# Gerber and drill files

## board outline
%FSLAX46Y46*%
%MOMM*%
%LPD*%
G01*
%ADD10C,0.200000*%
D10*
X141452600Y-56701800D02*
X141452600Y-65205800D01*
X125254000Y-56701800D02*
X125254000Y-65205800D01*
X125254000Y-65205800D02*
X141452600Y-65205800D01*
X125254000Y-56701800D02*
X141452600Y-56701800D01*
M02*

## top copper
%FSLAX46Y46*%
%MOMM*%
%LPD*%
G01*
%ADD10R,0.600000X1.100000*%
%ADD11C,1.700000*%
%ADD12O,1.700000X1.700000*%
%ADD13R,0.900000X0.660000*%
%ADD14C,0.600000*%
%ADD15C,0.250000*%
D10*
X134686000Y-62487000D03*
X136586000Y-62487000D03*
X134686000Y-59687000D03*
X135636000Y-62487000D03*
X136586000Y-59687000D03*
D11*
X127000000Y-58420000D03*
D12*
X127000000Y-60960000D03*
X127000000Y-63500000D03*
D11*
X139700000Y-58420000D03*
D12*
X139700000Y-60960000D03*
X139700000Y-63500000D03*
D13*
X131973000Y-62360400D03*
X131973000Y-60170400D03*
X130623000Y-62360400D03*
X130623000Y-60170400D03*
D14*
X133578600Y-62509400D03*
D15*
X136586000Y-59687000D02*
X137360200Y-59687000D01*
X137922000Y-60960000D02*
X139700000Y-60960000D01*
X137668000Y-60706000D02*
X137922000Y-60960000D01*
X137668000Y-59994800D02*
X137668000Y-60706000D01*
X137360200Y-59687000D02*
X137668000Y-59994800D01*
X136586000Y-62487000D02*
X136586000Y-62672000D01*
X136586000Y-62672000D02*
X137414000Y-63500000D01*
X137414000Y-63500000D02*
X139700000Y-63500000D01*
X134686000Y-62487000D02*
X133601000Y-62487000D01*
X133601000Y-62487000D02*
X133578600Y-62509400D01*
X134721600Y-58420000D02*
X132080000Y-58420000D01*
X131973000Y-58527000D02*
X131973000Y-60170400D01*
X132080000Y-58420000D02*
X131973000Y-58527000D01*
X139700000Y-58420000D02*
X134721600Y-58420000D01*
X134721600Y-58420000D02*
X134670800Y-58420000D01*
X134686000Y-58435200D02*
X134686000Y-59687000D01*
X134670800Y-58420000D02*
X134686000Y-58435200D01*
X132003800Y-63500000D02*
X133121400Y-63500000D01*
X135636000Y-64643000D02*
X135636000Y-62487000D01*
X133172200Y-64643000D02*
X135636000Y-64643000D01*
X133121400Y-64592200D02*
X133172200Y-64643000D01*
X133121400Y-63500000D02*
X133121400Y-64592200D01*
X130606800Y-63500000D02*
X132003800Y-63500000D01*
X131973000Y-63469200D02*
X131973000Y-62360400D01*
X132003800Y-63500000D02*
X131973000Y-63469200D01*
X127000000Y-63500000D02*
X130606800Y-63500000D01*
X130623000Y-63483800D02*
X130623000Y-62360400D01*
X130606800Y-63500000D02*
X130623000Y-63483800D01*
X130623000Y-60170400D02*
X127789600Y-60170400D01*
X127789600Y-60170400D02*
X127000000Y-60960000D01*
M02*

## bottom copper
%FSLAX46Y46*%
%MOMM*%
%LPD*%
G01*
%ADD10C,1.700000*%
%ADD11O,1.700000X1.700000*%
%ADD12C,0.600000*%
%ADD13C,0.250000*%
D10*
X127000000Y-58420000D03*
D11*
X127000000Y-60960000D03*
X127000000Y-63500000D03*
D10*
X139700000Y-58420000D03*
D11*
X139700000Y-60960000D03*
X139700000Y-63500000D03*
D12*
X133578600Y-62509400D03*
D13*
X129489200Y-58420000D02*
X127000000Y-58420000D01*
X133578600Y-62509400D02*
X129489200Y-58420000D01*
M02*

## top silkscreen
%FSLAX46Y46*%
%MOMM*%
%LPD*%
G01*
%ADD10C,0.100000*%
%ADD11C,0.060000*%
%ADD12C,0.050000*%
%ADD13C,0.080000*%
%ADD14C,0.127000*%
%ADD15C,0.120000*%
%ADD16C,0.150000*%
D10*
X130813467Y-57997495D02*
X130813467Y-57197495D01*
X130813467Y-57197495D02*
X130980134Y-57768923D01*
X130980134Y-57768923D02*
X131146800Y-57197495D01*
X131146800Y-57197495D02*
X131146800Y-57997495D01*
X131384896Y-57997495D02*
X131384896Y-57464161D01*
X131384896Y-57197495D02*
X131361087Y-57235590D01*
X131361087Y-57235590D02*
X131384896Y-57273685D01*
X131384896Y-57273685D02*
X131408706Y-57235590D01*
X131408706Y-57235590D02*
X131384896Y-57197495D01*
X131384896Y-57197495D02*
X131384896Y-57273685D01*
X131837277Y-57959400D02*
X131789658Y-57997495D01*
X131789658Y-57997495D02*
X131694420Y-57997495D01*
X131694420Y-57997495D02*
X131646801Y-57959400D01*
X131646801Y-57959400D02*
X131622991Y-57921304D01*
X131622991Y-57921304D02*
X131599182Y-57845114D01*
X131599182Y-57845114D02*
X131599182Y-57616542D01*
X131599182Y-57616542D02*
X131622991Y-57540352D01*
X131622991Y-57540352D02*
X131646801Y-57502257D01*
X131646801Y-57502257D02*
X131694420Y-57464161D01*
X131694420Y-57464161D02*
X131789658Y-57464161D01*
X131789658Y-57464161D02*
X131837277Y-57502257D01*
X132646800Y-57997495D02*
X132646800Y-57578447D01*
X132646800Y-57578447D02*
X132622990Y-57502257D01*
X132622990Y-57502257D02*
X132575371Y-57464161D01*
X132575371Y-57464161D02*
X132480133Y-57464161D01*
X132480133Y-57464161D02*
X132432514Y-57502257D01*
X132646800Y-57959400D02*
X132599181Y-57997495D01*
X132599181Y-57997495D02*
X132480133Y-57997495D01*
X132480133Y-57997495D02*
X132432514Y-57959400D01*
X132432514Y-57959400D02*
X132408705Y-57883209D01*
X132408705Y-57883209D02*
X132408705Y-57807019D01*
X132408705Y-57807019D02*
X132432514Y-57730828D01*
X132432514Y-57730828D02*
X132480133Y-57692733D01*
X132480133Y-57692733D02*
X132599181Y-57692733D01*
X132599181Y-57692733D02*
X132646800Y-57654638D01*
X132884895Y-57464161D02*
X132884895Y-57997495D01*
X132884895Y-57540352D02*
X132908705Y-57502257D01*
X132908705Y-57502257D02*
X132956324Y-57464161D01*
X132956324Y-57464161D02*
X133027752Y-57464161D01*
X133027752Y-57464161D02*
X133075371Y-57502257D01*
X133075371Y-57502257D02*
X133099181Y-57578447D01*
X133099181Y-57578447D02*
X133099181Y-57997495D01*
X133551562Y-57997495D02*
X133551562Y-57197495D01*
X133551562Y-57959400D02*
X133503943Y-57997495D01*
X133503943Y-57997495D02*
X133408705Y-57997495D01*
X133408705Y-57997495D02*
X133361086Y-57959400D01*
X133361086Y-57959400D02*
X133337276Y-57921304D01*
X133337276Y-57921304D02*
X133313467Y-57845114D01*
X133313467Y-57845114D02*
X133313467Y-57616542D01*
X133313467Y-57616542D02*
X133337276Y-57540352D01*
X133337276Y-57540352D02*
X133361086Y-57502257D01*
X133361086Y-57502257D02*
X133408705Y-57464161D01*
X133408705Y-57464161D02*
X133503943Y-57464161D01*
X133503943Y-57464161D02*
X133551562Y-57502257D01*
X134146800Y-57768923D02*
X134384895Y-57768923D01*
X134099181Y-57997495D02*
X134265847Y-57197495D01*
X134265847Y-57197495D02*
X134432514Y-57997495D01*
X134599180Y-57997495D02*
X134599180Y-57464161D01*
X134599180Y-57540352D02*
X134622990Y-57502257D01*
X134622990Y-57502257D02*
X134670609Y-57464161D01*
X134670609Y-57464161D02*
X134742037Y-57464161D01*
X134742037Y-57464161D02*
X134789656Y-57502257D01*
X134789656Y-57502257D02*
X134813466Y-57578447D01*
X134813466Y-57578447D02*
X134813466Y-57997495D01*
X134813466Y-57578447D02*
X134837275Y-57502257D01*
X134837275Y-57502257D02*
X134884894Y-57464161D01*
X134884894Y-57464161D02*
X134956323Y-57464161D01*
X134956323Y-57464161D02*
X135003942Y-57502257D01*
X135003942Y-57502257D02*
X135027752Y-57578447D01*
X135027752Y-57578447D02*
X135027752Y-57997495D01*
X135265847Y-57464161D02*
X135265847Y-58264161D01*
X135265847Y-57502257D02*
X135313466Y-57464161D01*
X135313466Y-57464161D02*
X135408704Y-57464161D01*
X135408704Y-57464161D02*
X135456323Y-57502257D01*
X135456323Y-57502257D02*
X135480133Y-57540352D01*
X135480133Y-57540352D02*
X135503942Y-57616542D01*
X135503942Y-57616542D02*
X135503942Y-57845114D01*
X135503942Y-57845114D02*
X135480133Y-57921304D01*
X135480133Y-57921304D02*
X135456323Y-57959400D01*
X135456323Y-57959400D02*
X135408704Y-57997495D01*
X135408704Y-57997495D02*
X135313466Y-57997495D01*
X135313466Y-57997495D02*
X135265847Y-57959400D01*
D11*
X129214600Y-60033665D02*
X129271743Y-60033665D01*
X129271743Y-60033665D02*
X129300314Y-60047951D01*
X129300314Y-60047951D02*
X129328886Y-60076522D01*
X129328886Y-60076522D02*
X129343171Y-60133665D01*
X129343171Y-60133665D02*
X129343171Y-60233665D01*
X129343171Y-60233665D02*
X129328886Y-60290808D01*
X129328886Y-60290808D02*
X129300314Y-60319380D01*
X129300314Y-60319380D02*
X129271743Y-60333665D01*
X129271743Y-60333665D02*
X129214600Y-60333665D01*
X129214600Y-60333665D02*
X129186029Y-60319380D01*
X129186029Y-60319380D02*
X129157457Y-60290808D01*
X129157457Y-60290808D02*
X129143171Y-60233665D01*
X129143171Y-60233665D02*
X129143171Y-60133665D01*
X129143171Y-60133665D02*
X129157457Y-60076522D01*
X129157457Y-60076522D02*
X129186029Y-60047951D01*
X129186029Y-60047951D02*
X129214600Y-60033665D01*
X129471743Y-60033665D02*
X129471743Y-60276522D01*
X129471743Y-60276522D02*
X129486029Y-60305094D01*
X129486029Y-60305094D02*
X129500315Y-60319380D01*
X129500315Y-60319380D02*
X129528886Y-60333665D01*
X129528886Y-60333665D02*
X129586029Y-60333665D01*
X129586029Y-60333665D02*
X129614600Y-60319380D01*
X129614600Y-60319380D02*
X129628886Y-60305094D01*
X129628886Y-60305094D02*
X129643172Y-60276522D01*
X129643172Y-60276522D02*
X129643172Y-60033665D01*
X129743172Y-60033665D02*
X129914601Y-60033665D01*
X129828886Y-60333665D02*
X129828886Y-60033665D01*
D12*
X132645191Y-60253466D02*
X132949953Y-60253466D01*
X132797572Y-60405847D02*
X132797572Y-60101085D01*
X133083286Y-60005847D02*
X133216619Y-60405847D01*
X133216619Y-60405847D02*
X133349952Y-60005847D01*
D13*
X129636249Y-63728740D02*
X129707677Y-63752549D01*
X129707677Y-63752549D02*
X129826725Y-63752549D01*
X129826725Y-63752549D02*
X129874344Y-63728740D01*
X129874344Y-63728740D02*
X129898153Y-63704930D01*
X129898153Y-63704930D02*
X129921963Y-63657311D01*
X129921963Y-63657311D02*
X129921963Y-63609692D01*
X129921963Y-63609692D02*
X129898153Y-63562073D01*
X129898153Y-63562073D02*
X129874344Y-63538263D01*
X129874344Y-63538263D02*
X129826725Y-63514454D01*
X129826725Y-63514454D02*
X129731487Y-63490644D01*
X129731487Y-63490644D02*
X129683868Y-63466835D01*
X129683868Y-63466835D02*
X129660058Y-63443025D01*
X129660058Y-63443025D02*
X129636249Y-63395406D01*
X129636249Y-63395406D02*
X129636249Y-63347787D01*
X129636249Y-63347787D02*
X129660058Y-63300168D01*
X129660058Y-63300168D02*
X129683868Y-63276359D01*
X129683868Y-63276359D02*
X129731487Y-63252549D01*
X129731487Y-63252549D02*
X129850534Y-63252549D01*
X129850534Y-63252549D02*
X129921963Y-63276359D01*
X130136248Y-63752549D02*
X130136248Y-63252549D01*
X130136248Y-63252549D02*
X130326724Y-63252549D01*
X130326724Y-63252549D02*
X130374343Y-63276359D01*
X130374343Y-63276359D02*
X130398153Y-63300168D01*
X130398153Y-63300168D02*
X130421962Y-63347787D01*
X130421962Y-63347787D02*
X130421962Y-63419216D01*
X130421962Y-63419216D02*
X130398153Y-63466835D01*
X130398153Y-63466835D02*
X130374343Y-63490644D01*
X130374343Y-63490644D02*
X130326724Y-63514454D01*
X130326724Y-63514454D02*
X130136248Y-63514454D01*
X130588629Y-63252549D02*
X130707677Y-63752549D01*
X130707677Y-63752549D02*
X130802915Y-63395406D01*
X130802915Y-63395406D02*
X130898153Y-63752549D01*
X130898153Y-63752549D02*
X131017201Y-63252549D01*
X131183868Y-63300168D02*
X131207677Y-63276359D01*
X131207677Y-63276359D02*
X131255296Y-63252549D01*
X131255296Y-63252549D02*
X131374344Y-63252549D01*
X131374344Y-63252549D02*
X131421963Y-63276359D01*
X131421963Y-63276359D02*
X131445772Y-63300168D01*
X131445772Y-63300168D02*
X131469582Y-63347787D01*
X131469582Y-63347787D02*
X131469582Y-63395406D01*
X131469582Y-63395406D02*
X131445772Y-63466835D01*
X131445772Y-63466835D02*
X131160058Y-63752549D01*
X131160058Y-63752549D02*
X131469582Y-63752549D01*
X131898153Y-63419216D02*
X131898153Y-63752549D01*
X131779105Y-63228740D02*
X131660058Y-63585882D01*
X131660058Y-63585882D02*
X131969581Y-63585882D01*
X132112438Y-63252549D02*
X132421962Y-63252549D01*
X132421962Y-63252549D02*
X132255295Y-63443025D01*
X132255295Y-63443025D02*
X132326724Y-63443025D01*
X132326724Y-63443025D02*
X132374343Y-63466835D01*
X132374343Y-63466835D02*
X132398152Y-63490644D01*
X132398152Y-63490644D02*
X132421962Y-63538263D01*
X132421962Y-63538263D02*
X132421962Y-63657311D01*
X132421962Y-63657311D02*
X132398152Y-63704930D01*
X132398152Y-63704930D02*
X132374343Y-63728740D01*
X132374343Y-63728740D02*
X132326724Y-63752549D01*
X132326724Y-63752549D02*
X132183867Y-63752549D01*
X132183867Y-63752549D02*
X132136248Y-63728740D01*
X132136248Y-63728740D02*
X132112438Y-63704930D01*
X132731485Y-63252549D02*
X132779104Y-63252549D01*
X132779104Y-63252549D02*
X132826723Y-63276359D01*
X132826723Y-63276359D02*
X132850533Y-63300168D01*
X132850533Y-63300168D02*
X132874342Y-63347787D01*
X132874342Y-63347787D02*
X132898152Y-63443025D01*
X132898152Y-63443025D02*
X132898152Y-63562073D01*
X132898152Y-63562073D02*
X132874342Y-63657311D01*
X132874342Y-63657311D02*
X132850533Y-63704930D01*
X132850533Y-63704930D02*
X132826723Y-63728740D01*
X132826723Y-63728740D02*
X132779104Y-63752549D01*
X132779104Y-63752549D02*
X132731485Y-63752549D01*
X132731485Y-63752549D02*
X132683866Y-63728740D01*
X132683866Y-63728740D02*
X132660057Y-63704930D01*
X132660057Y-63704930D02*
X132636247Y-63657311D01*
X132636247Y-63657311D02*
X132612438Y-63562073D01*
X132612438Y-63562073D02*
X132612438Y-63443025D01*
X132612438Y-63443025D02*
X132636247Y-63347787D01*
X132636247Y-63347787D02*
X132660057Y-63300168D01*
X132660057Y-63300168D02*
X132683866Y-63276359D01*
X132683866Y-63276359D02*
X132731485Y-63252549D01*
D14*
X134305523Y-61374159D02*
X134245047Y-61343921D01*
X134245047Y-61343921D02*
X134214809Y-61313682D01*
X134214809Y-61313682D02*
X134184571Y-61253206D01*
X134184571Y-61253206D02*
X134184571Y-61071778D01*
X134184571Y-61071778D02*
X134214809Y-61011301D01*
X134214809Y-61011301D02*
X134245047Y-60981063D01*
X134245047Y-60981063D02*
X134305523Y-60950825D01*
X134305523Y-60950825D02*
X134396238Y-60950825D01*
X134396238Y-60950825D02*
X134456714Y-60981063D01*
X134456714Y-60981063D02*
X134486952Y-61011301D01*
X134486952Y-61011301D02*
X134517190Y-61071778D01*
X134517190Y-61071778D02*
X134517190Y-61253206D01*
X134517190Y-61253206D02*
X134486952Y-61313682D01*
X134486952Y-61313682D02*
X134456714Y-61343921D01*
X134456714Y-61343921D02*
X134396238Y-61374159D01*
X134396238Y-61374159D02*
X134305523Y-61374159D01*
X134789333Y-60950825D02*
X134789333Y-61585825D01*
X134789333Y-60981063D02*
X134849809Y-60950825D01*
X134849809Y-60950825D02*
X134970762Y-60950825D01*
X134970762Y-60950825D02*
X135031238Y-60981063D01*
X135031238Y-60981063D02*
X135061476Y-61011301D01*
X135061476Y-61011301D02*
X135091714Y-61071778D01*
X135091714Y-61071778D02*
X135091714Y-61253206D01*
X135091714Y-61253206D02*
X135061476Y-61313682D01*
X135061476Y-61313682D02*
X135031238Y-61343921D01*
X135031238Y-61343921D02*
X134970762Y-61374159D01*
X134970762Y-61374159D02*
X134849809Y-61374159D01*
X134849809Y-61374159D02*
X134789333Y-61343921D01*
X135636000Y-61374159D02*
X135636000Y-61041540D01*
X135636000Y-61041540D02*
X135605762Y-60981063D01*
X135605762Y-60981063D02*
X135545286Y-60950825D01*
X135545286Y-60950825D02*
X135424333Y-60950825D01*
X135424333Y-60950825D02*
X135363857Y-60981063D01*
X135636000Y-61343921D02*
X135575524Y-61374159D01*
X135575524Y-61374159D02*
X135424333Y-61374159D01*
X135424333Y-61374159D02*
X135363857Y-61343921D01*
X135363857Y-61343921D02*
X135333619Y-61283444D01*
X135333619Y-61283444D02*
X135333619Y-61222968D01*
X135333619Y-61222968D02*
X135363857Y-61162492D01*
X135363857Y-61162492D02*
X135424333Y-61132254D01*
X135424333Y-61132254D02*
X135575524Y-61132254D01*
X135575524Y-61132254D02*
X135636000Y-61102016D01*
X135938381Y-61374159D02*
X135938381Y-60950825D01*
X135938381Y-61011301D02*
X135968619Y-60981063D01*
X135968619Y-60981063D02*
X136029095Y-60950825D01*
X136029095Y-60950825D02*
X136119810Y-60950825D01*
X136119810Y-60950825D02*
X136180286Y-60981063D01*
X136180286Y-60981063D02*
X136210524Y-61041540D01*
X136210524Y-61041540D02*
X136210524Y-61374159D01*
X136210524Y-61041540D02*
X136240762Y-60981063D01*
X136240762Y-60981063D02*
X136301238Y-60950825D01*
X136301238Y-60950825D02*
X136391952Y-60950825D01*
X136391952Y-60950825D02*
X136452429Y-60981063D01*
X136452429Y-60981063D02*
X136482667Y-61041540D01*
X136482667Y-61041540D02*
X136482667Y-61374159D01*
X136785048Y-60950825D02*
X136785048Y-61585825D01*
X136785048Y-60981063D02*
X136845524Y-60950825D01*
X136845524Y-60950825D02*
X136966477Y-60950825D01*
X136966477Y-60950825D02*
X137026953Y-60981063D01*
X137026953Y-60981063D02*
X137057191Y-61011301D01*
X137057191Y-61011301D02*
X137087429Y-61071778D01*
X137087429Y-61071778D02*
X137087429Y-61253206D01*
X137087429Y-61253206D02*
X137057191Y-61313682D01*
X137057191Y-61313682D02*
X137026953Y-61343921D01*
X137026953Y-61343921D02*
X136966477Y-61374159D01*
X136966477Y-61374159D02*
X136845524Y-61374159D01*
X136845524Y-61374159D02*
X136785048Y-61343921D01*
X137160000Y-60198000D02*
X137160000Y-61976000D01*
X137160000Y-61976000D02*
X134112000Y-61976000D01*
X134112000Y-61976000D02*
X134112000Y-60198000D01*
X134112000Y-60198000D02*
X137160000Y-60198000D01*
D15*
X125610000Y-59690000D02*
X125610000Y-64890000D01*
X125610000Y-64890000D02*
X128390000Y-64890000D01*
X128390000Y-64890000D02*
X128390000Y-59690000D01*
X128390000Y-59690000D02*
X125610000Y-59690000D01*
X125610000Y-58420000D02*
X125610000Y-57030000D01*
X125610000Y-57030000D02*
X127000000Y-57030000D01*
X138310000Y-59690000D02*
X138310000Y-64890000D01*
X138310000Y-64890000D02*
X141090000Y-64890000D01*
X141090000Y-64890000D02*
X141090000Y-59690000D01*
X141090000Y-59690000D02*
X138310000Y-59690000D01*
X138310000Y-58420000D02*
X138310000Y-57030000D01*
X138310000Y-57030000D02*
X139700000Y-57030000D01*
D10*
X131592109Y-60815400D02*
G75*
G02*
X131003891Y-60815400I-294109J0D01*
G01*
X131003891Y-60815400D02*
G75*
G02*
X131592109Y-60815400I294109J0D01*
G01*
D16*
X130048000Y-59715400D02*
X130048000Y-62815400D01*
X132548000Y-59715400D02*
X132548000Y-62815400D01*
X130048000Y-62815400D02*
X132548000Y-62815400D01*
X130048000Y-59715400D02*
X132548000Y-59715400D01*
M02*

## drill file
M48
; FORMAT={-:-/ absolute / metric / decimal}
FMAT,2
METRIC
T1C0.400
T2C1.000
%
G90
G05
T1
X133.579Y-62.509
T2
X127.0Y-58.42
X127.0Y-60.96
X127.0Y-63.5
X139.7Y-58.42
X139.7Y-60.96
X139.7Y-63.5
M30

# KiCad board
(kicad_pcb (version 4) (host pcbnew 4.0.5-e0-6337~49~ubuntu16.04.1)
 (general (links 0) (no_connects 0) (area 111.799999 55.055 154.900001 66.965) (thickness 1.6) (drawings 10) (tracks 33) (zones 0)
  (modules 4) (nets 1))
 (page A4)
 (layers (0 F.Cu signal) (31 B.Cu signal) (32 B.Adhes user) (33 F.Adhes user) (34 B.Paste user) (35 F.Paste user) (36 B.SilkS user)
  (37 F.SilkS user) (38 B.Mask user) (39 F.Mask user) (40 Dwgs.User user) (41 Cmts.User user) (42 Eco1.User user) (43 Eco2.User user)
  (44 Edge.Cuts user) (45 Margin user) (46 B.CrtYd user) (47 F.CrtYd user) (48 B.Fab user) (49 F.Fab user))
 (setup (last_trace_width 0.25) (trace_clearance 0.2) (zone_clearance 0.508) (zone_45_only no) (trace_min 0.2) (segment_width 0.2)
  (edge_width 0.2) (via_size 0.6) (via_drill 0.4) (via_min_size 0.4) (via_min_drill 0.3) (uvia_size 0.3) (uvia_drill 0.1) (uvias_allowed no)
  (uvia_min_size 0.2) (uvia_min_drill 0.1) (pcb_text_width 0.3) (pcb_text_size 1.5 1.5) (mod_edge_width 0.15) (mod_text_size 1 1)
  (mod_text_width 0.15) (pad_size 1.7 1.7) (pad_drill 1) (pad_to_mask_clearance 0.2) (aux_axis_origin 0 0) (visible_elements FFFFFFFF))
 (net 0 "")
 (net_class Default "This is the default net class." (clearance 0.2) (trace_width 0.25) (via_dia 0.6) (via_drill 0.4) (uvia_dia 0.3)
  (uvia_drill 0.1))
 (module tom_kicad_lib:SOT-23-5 (layer F.Cu) (at 135.636 61.087) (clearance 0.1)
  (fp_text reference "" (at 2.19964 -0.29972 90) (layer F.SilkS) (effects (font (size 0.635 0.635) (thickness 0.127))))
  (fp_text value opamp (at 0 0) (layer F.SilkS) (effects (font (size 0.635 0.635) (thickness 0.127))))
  (fp_line (start 1.524 -0.889) (end 1.524 0.889) (layer F.SilkS) (width 0.127))
  (fp_line (start 1.524 0.889) (end -1.524 0.889) (layer F.SilkS) (width 0.127))
  (fp_line (start -1.524 0.889) (end -1.524 -0.889) (layer F.SilkS) (width 0.127))
  (fp_line (start -1.524 -0.889) (end 1.524 -0.889) (layer F.SilkS) (width 0.127))
  (pad 1 smd rect (at -0.95 1.4) (size 0.6 1.1) (layers F.Cu F.Paste F.Mask))
  (pad 3 smd rect (at 0.95 1.4) (size 0.6 1.1) (layers F.Cu F.Paste F.Mask))
  (pad 5 smd rect (at -0.95 -1.4) (size 0.6 1.1) (layers F.Cu F.Paste F.Mask))
  (pad 2 smd rect (at 0 1.4) (size 0.6 1.1) (layers F.Cu F.Paste F.Mask))
  (pad 4 smd rect (at 0.95 -1.4) (size 0.6 1.1) (layers F.Cu F.Paste F.Mask)))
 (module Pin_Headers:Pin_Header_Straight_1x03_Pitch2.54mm (layer F.Cu) (at 127 58.42)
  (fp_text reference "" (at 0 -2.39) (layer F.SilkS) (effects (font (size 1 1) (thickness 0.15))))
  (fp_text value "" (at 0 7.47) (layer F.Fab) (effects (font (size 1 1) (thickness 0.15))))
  (fp_line (start -1.39 1.27) (end -1.39 6.47) (layer F.SilkS) (width 0.12))
  (fp_line (start -1.39 6.47) (end 1.39 6.47) (layer F.SilkS) (width 0.12))
  (fp_line (start 1.39 6.47) (end 1.39 1.27) (layer F.SilkS) (width 0.12))
  (fp_line (start 1.39 1.27) (end -1.39 1.27) (layer F.SilkS) (width 0.12))
  (fp_line (start -1.39 0) (end -1.39 -1.39) (layer F.SilkS) (width 0.12))
  (fp_line (start -1.39 -1.39) (end 0 -1.39) (layer F.SilkS) (width 0.12))
  (pad 1 thru_hole circle (at 0 0) (size 1.7 1.7) (drill 1) (layers *.Cu *.Mask))
  (pad 2 thru_hole oval (at 0 2.54) (size 1.7 1.7) (drill 1) (layers *.Cu *.Mask))
  (pad 3 thru_hole oval (at 0 5.08) (size 1.7 1.7) (drill 1) (layers *.Cu *.Mask)))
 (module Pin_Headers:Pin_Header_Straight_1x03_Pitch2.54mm (layer F.Cu) (at 139.7 58.42)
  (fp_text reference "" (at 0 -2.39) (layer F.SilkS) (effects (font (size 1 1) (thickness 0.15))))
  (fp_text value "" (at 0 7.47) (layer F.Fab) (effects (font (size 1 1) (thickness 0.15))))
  (fp_line (start -1.39 1.27) (end -1.39 6.47) (layer F.SilkS) (width 0.12))
  (fp_line (start -1.39 6.47) (end 1.39 6.47) (layer F.SilkS) (width 0.12))
  (fp_line (start 1.39 6.47) (end 1.39 1.27) (layer F.SilkS) (width 0.12))
  (fp_line (start 1.39 1.27) (end -1.39 1.27) (layer F.SilkS) (width 0.12))
  (fp_line (start -1.39 0) (end -1.39 -1.39) (layer F.SilkS) (width 0.12))
  (fp_line (start -1.39 -1.39) (end 0 -1.39) (layer F.SilkS) (width 0.12))
  (pad 1 thru_hole circle (at 0 0) (size 1.7 1.7) (drill 1) (layers *.Cu *.Mask))
  (pad 2 thru_hole oval (at 0 2.54) (size 1.7 1.7) (drill 1) (layers *.Cu *.Mask))
  (pad 3 thru_hole oval (at 0 5.08) (size 1.7 1.7) (drill 1) (layers *.Cu *.Mask)))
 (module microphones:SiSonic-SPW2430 (layer F.Cu) (at 130.048 59.7154)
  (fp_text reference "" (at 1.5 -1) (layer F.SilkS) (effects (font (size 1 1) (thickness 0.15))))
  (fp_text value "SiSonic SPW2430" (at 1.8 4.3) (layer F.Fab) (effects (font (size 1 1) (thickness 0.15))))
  (fp_circle (center 1.25 1.1) (end 1.53 1.19) (layer F.SilkS) (width 0.1))
  (fp_line (start 0 0) (end 0 3.1) (layer F.SilkS) (width 0.15))
  (fp_line (start 2.5 0) (end 2.5 3.1) (layer F.SilkS) (width 0.15))
  (fp_line (start 0 3.1) (end 2.5 3.1) (layer F.SilkS) (width 0.15))
  (fp_line (start 0 0) (end 2.5 0) (layer F.SilkS) (width 0.15))
  (pad GND smd rect (at 1.925 2.645) (size 0.9 0.66) (layers F.Cu F.Paste F.Mask))
  (pad +V smd rect (at 1.925 0.455) (size 0.9 0.66) (layers F.Cu F.Paste F.Mask))
  (pad GND smd rect (at 0.575 2.645) (size 0.9 0.66) (layers F.Cu F.Paste F.Mask))
  (pad OUT smd rect (at 0.575 0.455) (size 0.9 0.66) (layers F.Cu F.Paste F.Mask)))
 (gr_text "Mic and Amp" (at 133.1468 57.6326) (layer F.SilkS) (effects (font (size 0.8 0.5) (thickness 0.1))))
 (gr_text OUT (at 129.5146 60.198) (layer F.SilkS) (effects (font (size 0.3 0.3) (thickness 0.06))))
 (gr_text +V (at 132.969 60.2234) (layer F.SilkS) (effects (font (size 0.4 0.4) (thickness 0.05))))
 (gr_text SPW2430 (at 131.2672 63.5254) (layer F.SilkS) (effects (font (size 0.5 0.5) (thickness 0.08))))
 (gr_line (start 141.4526 56.7018) (end 141.4526 65.2058) (angle 90) (layer Edge.Cuts) (width 0.2))
 (gr_line (start 125.254 56.7018) (end 125.254 65.2058) (angle 90) (layer Edge.Cuts) (width 0.2))
 (gr_line (start 125.254 65.2058) (end 141.4526 65.2058) (angle 90) (layer Edge.Cuts) (width 0.2))
 (gr_line (start 125.254 56.7018) (end 141.4526 56.7018) (angle 90) (layer Edge.Cuts) (width 0.2))
 (segment (start 136.586 59.687) (end 137.3602 59.687) (width 0.25) (layer F.Cu) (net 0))
 (segment (start 137.922 60.96) (end 139.7 60.96) (width 0.25) (layer F.Cu) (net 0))
 (segment (start 137.668 60.706) (end 137.922 60.96) (width 0.25) (layer F.Cu) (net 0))
 (segment (start 137.668 59.9948) (end 137.668 60.706) (width 0.25) (layer F.Cu) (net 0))
 (segment (start 137.3602 59.687) (end 137.668 59.9948) (width 0.25) (layer F.Cu) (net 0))
 (segment (start 136.586 62.487) (end 136.586 62.672) (width 0.25) (layer F.Cu) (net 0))
 (segment (start 136.586 62.672) (end 137.414 63.5) (width 0.25) (layer F.Cu) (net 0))
 (segment (start 137.414 63.5) (end 139.7 63.5) (width 0.25) (layer F.Cu) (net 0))
 (segment (start 134.686 62.487) (end 133.601 62.487) (width 0.25) (layer F.Cu) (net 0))
 (segment (start 129.4892 58.42) (end 127 58.42) (width 0.25) (layer B.Cu) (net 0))
 (segment (start 133.5786 62.5094) (end 129.4892 58.42) (width 0.25) (layer B.Cu) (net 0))
 (via (at 133.5786 62.5094) (size 0.6) (drill 0.4) (layers F.Cu B.Cu) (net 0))
 (segment (start 133.601 62.487) (end 133.5786 62.5094) (width 0.25) (layer F.Cu) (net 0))
 (segment (start 134.7216 58.42) (end 132.08 58.42) (width 0.25) (layer F.Cu) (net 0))
 (segment (start 131.973 58.527) (end 131.973 60.1704) (width 0.25) (layer F.Cu) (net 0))
 (segment (start 132.08 58.42) (end 131.973 58.527) (width 0.25) (layer F.Cu) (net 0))
 (segment (start 139.7 58.42) (end 134.7216 58.42) (width 0.25) (layer F.Cu) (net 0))
 (segment (start 134.7216 58.42) (end 134.6708 58.42) (width 0.25) (layer F.Cu) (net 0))
 (segment (start 134.686 58.4352) (end 134.686 59.687) (width 0.25) (layer F.Cu) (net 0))
 (segment (start 134.6708 58.42) (end 134.686 58.4352) (width 0.25) (layer F.Cu) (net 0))
 (segment (start 132.0038 63.5) (end 133.1214 63.5) (width 0.25) (layer F.Cu) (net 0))
 (segment (start 135.636 64.643) (end 135.636 62.487) (width 0.25) (layer F.Cu) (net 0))
 (segment (start 133.1722 64.643) (end 135.636 64.643) (width 0.25) (layer F.Cu) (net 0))
 (segment (start 133.1214 64.5922) (end 133.1722 64.643) (width 0.25) (layer F.Cu) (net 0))
 (segment (start 133.1214 63.5) (end 133.1214 64.5922) (width 0.25) (layer F.Cu) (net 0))
 (segment (start 130.6068 63.5) (end 132.0038 63.5) (width 0.25) (layer F.Cu) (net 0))
 (segment (start 131.973 63.4692) (end 131.973 62.3604) (width 0.25) (layer F.Cu) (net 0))
 (segment (start 132.0038 63.5) (end 131.973 63.4692) (width 0.25) (layer F.Cu) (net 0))
 (segment (start 127 63.5) (end 130.6068 63.5) (width 0.25) (layer F.Cu) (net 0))
 (segment (start 130.623 63.4838) (end 130.623 62.3604) (width 0.25) (layer F.Cu) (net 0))
 (segment (start 130.6068 63.5) (end 130.623 63.4838) (width 0.25) (layer F.Cu) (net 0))
 (segment (start 130.623 60.1704) (end 127.7896 60.1704) (width 0.25) (layer F.Cu) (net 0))
 (segment (start 127.7896 60.1704) (end 127 60.96) (width 0.25) (layer F.Cu) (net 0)))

